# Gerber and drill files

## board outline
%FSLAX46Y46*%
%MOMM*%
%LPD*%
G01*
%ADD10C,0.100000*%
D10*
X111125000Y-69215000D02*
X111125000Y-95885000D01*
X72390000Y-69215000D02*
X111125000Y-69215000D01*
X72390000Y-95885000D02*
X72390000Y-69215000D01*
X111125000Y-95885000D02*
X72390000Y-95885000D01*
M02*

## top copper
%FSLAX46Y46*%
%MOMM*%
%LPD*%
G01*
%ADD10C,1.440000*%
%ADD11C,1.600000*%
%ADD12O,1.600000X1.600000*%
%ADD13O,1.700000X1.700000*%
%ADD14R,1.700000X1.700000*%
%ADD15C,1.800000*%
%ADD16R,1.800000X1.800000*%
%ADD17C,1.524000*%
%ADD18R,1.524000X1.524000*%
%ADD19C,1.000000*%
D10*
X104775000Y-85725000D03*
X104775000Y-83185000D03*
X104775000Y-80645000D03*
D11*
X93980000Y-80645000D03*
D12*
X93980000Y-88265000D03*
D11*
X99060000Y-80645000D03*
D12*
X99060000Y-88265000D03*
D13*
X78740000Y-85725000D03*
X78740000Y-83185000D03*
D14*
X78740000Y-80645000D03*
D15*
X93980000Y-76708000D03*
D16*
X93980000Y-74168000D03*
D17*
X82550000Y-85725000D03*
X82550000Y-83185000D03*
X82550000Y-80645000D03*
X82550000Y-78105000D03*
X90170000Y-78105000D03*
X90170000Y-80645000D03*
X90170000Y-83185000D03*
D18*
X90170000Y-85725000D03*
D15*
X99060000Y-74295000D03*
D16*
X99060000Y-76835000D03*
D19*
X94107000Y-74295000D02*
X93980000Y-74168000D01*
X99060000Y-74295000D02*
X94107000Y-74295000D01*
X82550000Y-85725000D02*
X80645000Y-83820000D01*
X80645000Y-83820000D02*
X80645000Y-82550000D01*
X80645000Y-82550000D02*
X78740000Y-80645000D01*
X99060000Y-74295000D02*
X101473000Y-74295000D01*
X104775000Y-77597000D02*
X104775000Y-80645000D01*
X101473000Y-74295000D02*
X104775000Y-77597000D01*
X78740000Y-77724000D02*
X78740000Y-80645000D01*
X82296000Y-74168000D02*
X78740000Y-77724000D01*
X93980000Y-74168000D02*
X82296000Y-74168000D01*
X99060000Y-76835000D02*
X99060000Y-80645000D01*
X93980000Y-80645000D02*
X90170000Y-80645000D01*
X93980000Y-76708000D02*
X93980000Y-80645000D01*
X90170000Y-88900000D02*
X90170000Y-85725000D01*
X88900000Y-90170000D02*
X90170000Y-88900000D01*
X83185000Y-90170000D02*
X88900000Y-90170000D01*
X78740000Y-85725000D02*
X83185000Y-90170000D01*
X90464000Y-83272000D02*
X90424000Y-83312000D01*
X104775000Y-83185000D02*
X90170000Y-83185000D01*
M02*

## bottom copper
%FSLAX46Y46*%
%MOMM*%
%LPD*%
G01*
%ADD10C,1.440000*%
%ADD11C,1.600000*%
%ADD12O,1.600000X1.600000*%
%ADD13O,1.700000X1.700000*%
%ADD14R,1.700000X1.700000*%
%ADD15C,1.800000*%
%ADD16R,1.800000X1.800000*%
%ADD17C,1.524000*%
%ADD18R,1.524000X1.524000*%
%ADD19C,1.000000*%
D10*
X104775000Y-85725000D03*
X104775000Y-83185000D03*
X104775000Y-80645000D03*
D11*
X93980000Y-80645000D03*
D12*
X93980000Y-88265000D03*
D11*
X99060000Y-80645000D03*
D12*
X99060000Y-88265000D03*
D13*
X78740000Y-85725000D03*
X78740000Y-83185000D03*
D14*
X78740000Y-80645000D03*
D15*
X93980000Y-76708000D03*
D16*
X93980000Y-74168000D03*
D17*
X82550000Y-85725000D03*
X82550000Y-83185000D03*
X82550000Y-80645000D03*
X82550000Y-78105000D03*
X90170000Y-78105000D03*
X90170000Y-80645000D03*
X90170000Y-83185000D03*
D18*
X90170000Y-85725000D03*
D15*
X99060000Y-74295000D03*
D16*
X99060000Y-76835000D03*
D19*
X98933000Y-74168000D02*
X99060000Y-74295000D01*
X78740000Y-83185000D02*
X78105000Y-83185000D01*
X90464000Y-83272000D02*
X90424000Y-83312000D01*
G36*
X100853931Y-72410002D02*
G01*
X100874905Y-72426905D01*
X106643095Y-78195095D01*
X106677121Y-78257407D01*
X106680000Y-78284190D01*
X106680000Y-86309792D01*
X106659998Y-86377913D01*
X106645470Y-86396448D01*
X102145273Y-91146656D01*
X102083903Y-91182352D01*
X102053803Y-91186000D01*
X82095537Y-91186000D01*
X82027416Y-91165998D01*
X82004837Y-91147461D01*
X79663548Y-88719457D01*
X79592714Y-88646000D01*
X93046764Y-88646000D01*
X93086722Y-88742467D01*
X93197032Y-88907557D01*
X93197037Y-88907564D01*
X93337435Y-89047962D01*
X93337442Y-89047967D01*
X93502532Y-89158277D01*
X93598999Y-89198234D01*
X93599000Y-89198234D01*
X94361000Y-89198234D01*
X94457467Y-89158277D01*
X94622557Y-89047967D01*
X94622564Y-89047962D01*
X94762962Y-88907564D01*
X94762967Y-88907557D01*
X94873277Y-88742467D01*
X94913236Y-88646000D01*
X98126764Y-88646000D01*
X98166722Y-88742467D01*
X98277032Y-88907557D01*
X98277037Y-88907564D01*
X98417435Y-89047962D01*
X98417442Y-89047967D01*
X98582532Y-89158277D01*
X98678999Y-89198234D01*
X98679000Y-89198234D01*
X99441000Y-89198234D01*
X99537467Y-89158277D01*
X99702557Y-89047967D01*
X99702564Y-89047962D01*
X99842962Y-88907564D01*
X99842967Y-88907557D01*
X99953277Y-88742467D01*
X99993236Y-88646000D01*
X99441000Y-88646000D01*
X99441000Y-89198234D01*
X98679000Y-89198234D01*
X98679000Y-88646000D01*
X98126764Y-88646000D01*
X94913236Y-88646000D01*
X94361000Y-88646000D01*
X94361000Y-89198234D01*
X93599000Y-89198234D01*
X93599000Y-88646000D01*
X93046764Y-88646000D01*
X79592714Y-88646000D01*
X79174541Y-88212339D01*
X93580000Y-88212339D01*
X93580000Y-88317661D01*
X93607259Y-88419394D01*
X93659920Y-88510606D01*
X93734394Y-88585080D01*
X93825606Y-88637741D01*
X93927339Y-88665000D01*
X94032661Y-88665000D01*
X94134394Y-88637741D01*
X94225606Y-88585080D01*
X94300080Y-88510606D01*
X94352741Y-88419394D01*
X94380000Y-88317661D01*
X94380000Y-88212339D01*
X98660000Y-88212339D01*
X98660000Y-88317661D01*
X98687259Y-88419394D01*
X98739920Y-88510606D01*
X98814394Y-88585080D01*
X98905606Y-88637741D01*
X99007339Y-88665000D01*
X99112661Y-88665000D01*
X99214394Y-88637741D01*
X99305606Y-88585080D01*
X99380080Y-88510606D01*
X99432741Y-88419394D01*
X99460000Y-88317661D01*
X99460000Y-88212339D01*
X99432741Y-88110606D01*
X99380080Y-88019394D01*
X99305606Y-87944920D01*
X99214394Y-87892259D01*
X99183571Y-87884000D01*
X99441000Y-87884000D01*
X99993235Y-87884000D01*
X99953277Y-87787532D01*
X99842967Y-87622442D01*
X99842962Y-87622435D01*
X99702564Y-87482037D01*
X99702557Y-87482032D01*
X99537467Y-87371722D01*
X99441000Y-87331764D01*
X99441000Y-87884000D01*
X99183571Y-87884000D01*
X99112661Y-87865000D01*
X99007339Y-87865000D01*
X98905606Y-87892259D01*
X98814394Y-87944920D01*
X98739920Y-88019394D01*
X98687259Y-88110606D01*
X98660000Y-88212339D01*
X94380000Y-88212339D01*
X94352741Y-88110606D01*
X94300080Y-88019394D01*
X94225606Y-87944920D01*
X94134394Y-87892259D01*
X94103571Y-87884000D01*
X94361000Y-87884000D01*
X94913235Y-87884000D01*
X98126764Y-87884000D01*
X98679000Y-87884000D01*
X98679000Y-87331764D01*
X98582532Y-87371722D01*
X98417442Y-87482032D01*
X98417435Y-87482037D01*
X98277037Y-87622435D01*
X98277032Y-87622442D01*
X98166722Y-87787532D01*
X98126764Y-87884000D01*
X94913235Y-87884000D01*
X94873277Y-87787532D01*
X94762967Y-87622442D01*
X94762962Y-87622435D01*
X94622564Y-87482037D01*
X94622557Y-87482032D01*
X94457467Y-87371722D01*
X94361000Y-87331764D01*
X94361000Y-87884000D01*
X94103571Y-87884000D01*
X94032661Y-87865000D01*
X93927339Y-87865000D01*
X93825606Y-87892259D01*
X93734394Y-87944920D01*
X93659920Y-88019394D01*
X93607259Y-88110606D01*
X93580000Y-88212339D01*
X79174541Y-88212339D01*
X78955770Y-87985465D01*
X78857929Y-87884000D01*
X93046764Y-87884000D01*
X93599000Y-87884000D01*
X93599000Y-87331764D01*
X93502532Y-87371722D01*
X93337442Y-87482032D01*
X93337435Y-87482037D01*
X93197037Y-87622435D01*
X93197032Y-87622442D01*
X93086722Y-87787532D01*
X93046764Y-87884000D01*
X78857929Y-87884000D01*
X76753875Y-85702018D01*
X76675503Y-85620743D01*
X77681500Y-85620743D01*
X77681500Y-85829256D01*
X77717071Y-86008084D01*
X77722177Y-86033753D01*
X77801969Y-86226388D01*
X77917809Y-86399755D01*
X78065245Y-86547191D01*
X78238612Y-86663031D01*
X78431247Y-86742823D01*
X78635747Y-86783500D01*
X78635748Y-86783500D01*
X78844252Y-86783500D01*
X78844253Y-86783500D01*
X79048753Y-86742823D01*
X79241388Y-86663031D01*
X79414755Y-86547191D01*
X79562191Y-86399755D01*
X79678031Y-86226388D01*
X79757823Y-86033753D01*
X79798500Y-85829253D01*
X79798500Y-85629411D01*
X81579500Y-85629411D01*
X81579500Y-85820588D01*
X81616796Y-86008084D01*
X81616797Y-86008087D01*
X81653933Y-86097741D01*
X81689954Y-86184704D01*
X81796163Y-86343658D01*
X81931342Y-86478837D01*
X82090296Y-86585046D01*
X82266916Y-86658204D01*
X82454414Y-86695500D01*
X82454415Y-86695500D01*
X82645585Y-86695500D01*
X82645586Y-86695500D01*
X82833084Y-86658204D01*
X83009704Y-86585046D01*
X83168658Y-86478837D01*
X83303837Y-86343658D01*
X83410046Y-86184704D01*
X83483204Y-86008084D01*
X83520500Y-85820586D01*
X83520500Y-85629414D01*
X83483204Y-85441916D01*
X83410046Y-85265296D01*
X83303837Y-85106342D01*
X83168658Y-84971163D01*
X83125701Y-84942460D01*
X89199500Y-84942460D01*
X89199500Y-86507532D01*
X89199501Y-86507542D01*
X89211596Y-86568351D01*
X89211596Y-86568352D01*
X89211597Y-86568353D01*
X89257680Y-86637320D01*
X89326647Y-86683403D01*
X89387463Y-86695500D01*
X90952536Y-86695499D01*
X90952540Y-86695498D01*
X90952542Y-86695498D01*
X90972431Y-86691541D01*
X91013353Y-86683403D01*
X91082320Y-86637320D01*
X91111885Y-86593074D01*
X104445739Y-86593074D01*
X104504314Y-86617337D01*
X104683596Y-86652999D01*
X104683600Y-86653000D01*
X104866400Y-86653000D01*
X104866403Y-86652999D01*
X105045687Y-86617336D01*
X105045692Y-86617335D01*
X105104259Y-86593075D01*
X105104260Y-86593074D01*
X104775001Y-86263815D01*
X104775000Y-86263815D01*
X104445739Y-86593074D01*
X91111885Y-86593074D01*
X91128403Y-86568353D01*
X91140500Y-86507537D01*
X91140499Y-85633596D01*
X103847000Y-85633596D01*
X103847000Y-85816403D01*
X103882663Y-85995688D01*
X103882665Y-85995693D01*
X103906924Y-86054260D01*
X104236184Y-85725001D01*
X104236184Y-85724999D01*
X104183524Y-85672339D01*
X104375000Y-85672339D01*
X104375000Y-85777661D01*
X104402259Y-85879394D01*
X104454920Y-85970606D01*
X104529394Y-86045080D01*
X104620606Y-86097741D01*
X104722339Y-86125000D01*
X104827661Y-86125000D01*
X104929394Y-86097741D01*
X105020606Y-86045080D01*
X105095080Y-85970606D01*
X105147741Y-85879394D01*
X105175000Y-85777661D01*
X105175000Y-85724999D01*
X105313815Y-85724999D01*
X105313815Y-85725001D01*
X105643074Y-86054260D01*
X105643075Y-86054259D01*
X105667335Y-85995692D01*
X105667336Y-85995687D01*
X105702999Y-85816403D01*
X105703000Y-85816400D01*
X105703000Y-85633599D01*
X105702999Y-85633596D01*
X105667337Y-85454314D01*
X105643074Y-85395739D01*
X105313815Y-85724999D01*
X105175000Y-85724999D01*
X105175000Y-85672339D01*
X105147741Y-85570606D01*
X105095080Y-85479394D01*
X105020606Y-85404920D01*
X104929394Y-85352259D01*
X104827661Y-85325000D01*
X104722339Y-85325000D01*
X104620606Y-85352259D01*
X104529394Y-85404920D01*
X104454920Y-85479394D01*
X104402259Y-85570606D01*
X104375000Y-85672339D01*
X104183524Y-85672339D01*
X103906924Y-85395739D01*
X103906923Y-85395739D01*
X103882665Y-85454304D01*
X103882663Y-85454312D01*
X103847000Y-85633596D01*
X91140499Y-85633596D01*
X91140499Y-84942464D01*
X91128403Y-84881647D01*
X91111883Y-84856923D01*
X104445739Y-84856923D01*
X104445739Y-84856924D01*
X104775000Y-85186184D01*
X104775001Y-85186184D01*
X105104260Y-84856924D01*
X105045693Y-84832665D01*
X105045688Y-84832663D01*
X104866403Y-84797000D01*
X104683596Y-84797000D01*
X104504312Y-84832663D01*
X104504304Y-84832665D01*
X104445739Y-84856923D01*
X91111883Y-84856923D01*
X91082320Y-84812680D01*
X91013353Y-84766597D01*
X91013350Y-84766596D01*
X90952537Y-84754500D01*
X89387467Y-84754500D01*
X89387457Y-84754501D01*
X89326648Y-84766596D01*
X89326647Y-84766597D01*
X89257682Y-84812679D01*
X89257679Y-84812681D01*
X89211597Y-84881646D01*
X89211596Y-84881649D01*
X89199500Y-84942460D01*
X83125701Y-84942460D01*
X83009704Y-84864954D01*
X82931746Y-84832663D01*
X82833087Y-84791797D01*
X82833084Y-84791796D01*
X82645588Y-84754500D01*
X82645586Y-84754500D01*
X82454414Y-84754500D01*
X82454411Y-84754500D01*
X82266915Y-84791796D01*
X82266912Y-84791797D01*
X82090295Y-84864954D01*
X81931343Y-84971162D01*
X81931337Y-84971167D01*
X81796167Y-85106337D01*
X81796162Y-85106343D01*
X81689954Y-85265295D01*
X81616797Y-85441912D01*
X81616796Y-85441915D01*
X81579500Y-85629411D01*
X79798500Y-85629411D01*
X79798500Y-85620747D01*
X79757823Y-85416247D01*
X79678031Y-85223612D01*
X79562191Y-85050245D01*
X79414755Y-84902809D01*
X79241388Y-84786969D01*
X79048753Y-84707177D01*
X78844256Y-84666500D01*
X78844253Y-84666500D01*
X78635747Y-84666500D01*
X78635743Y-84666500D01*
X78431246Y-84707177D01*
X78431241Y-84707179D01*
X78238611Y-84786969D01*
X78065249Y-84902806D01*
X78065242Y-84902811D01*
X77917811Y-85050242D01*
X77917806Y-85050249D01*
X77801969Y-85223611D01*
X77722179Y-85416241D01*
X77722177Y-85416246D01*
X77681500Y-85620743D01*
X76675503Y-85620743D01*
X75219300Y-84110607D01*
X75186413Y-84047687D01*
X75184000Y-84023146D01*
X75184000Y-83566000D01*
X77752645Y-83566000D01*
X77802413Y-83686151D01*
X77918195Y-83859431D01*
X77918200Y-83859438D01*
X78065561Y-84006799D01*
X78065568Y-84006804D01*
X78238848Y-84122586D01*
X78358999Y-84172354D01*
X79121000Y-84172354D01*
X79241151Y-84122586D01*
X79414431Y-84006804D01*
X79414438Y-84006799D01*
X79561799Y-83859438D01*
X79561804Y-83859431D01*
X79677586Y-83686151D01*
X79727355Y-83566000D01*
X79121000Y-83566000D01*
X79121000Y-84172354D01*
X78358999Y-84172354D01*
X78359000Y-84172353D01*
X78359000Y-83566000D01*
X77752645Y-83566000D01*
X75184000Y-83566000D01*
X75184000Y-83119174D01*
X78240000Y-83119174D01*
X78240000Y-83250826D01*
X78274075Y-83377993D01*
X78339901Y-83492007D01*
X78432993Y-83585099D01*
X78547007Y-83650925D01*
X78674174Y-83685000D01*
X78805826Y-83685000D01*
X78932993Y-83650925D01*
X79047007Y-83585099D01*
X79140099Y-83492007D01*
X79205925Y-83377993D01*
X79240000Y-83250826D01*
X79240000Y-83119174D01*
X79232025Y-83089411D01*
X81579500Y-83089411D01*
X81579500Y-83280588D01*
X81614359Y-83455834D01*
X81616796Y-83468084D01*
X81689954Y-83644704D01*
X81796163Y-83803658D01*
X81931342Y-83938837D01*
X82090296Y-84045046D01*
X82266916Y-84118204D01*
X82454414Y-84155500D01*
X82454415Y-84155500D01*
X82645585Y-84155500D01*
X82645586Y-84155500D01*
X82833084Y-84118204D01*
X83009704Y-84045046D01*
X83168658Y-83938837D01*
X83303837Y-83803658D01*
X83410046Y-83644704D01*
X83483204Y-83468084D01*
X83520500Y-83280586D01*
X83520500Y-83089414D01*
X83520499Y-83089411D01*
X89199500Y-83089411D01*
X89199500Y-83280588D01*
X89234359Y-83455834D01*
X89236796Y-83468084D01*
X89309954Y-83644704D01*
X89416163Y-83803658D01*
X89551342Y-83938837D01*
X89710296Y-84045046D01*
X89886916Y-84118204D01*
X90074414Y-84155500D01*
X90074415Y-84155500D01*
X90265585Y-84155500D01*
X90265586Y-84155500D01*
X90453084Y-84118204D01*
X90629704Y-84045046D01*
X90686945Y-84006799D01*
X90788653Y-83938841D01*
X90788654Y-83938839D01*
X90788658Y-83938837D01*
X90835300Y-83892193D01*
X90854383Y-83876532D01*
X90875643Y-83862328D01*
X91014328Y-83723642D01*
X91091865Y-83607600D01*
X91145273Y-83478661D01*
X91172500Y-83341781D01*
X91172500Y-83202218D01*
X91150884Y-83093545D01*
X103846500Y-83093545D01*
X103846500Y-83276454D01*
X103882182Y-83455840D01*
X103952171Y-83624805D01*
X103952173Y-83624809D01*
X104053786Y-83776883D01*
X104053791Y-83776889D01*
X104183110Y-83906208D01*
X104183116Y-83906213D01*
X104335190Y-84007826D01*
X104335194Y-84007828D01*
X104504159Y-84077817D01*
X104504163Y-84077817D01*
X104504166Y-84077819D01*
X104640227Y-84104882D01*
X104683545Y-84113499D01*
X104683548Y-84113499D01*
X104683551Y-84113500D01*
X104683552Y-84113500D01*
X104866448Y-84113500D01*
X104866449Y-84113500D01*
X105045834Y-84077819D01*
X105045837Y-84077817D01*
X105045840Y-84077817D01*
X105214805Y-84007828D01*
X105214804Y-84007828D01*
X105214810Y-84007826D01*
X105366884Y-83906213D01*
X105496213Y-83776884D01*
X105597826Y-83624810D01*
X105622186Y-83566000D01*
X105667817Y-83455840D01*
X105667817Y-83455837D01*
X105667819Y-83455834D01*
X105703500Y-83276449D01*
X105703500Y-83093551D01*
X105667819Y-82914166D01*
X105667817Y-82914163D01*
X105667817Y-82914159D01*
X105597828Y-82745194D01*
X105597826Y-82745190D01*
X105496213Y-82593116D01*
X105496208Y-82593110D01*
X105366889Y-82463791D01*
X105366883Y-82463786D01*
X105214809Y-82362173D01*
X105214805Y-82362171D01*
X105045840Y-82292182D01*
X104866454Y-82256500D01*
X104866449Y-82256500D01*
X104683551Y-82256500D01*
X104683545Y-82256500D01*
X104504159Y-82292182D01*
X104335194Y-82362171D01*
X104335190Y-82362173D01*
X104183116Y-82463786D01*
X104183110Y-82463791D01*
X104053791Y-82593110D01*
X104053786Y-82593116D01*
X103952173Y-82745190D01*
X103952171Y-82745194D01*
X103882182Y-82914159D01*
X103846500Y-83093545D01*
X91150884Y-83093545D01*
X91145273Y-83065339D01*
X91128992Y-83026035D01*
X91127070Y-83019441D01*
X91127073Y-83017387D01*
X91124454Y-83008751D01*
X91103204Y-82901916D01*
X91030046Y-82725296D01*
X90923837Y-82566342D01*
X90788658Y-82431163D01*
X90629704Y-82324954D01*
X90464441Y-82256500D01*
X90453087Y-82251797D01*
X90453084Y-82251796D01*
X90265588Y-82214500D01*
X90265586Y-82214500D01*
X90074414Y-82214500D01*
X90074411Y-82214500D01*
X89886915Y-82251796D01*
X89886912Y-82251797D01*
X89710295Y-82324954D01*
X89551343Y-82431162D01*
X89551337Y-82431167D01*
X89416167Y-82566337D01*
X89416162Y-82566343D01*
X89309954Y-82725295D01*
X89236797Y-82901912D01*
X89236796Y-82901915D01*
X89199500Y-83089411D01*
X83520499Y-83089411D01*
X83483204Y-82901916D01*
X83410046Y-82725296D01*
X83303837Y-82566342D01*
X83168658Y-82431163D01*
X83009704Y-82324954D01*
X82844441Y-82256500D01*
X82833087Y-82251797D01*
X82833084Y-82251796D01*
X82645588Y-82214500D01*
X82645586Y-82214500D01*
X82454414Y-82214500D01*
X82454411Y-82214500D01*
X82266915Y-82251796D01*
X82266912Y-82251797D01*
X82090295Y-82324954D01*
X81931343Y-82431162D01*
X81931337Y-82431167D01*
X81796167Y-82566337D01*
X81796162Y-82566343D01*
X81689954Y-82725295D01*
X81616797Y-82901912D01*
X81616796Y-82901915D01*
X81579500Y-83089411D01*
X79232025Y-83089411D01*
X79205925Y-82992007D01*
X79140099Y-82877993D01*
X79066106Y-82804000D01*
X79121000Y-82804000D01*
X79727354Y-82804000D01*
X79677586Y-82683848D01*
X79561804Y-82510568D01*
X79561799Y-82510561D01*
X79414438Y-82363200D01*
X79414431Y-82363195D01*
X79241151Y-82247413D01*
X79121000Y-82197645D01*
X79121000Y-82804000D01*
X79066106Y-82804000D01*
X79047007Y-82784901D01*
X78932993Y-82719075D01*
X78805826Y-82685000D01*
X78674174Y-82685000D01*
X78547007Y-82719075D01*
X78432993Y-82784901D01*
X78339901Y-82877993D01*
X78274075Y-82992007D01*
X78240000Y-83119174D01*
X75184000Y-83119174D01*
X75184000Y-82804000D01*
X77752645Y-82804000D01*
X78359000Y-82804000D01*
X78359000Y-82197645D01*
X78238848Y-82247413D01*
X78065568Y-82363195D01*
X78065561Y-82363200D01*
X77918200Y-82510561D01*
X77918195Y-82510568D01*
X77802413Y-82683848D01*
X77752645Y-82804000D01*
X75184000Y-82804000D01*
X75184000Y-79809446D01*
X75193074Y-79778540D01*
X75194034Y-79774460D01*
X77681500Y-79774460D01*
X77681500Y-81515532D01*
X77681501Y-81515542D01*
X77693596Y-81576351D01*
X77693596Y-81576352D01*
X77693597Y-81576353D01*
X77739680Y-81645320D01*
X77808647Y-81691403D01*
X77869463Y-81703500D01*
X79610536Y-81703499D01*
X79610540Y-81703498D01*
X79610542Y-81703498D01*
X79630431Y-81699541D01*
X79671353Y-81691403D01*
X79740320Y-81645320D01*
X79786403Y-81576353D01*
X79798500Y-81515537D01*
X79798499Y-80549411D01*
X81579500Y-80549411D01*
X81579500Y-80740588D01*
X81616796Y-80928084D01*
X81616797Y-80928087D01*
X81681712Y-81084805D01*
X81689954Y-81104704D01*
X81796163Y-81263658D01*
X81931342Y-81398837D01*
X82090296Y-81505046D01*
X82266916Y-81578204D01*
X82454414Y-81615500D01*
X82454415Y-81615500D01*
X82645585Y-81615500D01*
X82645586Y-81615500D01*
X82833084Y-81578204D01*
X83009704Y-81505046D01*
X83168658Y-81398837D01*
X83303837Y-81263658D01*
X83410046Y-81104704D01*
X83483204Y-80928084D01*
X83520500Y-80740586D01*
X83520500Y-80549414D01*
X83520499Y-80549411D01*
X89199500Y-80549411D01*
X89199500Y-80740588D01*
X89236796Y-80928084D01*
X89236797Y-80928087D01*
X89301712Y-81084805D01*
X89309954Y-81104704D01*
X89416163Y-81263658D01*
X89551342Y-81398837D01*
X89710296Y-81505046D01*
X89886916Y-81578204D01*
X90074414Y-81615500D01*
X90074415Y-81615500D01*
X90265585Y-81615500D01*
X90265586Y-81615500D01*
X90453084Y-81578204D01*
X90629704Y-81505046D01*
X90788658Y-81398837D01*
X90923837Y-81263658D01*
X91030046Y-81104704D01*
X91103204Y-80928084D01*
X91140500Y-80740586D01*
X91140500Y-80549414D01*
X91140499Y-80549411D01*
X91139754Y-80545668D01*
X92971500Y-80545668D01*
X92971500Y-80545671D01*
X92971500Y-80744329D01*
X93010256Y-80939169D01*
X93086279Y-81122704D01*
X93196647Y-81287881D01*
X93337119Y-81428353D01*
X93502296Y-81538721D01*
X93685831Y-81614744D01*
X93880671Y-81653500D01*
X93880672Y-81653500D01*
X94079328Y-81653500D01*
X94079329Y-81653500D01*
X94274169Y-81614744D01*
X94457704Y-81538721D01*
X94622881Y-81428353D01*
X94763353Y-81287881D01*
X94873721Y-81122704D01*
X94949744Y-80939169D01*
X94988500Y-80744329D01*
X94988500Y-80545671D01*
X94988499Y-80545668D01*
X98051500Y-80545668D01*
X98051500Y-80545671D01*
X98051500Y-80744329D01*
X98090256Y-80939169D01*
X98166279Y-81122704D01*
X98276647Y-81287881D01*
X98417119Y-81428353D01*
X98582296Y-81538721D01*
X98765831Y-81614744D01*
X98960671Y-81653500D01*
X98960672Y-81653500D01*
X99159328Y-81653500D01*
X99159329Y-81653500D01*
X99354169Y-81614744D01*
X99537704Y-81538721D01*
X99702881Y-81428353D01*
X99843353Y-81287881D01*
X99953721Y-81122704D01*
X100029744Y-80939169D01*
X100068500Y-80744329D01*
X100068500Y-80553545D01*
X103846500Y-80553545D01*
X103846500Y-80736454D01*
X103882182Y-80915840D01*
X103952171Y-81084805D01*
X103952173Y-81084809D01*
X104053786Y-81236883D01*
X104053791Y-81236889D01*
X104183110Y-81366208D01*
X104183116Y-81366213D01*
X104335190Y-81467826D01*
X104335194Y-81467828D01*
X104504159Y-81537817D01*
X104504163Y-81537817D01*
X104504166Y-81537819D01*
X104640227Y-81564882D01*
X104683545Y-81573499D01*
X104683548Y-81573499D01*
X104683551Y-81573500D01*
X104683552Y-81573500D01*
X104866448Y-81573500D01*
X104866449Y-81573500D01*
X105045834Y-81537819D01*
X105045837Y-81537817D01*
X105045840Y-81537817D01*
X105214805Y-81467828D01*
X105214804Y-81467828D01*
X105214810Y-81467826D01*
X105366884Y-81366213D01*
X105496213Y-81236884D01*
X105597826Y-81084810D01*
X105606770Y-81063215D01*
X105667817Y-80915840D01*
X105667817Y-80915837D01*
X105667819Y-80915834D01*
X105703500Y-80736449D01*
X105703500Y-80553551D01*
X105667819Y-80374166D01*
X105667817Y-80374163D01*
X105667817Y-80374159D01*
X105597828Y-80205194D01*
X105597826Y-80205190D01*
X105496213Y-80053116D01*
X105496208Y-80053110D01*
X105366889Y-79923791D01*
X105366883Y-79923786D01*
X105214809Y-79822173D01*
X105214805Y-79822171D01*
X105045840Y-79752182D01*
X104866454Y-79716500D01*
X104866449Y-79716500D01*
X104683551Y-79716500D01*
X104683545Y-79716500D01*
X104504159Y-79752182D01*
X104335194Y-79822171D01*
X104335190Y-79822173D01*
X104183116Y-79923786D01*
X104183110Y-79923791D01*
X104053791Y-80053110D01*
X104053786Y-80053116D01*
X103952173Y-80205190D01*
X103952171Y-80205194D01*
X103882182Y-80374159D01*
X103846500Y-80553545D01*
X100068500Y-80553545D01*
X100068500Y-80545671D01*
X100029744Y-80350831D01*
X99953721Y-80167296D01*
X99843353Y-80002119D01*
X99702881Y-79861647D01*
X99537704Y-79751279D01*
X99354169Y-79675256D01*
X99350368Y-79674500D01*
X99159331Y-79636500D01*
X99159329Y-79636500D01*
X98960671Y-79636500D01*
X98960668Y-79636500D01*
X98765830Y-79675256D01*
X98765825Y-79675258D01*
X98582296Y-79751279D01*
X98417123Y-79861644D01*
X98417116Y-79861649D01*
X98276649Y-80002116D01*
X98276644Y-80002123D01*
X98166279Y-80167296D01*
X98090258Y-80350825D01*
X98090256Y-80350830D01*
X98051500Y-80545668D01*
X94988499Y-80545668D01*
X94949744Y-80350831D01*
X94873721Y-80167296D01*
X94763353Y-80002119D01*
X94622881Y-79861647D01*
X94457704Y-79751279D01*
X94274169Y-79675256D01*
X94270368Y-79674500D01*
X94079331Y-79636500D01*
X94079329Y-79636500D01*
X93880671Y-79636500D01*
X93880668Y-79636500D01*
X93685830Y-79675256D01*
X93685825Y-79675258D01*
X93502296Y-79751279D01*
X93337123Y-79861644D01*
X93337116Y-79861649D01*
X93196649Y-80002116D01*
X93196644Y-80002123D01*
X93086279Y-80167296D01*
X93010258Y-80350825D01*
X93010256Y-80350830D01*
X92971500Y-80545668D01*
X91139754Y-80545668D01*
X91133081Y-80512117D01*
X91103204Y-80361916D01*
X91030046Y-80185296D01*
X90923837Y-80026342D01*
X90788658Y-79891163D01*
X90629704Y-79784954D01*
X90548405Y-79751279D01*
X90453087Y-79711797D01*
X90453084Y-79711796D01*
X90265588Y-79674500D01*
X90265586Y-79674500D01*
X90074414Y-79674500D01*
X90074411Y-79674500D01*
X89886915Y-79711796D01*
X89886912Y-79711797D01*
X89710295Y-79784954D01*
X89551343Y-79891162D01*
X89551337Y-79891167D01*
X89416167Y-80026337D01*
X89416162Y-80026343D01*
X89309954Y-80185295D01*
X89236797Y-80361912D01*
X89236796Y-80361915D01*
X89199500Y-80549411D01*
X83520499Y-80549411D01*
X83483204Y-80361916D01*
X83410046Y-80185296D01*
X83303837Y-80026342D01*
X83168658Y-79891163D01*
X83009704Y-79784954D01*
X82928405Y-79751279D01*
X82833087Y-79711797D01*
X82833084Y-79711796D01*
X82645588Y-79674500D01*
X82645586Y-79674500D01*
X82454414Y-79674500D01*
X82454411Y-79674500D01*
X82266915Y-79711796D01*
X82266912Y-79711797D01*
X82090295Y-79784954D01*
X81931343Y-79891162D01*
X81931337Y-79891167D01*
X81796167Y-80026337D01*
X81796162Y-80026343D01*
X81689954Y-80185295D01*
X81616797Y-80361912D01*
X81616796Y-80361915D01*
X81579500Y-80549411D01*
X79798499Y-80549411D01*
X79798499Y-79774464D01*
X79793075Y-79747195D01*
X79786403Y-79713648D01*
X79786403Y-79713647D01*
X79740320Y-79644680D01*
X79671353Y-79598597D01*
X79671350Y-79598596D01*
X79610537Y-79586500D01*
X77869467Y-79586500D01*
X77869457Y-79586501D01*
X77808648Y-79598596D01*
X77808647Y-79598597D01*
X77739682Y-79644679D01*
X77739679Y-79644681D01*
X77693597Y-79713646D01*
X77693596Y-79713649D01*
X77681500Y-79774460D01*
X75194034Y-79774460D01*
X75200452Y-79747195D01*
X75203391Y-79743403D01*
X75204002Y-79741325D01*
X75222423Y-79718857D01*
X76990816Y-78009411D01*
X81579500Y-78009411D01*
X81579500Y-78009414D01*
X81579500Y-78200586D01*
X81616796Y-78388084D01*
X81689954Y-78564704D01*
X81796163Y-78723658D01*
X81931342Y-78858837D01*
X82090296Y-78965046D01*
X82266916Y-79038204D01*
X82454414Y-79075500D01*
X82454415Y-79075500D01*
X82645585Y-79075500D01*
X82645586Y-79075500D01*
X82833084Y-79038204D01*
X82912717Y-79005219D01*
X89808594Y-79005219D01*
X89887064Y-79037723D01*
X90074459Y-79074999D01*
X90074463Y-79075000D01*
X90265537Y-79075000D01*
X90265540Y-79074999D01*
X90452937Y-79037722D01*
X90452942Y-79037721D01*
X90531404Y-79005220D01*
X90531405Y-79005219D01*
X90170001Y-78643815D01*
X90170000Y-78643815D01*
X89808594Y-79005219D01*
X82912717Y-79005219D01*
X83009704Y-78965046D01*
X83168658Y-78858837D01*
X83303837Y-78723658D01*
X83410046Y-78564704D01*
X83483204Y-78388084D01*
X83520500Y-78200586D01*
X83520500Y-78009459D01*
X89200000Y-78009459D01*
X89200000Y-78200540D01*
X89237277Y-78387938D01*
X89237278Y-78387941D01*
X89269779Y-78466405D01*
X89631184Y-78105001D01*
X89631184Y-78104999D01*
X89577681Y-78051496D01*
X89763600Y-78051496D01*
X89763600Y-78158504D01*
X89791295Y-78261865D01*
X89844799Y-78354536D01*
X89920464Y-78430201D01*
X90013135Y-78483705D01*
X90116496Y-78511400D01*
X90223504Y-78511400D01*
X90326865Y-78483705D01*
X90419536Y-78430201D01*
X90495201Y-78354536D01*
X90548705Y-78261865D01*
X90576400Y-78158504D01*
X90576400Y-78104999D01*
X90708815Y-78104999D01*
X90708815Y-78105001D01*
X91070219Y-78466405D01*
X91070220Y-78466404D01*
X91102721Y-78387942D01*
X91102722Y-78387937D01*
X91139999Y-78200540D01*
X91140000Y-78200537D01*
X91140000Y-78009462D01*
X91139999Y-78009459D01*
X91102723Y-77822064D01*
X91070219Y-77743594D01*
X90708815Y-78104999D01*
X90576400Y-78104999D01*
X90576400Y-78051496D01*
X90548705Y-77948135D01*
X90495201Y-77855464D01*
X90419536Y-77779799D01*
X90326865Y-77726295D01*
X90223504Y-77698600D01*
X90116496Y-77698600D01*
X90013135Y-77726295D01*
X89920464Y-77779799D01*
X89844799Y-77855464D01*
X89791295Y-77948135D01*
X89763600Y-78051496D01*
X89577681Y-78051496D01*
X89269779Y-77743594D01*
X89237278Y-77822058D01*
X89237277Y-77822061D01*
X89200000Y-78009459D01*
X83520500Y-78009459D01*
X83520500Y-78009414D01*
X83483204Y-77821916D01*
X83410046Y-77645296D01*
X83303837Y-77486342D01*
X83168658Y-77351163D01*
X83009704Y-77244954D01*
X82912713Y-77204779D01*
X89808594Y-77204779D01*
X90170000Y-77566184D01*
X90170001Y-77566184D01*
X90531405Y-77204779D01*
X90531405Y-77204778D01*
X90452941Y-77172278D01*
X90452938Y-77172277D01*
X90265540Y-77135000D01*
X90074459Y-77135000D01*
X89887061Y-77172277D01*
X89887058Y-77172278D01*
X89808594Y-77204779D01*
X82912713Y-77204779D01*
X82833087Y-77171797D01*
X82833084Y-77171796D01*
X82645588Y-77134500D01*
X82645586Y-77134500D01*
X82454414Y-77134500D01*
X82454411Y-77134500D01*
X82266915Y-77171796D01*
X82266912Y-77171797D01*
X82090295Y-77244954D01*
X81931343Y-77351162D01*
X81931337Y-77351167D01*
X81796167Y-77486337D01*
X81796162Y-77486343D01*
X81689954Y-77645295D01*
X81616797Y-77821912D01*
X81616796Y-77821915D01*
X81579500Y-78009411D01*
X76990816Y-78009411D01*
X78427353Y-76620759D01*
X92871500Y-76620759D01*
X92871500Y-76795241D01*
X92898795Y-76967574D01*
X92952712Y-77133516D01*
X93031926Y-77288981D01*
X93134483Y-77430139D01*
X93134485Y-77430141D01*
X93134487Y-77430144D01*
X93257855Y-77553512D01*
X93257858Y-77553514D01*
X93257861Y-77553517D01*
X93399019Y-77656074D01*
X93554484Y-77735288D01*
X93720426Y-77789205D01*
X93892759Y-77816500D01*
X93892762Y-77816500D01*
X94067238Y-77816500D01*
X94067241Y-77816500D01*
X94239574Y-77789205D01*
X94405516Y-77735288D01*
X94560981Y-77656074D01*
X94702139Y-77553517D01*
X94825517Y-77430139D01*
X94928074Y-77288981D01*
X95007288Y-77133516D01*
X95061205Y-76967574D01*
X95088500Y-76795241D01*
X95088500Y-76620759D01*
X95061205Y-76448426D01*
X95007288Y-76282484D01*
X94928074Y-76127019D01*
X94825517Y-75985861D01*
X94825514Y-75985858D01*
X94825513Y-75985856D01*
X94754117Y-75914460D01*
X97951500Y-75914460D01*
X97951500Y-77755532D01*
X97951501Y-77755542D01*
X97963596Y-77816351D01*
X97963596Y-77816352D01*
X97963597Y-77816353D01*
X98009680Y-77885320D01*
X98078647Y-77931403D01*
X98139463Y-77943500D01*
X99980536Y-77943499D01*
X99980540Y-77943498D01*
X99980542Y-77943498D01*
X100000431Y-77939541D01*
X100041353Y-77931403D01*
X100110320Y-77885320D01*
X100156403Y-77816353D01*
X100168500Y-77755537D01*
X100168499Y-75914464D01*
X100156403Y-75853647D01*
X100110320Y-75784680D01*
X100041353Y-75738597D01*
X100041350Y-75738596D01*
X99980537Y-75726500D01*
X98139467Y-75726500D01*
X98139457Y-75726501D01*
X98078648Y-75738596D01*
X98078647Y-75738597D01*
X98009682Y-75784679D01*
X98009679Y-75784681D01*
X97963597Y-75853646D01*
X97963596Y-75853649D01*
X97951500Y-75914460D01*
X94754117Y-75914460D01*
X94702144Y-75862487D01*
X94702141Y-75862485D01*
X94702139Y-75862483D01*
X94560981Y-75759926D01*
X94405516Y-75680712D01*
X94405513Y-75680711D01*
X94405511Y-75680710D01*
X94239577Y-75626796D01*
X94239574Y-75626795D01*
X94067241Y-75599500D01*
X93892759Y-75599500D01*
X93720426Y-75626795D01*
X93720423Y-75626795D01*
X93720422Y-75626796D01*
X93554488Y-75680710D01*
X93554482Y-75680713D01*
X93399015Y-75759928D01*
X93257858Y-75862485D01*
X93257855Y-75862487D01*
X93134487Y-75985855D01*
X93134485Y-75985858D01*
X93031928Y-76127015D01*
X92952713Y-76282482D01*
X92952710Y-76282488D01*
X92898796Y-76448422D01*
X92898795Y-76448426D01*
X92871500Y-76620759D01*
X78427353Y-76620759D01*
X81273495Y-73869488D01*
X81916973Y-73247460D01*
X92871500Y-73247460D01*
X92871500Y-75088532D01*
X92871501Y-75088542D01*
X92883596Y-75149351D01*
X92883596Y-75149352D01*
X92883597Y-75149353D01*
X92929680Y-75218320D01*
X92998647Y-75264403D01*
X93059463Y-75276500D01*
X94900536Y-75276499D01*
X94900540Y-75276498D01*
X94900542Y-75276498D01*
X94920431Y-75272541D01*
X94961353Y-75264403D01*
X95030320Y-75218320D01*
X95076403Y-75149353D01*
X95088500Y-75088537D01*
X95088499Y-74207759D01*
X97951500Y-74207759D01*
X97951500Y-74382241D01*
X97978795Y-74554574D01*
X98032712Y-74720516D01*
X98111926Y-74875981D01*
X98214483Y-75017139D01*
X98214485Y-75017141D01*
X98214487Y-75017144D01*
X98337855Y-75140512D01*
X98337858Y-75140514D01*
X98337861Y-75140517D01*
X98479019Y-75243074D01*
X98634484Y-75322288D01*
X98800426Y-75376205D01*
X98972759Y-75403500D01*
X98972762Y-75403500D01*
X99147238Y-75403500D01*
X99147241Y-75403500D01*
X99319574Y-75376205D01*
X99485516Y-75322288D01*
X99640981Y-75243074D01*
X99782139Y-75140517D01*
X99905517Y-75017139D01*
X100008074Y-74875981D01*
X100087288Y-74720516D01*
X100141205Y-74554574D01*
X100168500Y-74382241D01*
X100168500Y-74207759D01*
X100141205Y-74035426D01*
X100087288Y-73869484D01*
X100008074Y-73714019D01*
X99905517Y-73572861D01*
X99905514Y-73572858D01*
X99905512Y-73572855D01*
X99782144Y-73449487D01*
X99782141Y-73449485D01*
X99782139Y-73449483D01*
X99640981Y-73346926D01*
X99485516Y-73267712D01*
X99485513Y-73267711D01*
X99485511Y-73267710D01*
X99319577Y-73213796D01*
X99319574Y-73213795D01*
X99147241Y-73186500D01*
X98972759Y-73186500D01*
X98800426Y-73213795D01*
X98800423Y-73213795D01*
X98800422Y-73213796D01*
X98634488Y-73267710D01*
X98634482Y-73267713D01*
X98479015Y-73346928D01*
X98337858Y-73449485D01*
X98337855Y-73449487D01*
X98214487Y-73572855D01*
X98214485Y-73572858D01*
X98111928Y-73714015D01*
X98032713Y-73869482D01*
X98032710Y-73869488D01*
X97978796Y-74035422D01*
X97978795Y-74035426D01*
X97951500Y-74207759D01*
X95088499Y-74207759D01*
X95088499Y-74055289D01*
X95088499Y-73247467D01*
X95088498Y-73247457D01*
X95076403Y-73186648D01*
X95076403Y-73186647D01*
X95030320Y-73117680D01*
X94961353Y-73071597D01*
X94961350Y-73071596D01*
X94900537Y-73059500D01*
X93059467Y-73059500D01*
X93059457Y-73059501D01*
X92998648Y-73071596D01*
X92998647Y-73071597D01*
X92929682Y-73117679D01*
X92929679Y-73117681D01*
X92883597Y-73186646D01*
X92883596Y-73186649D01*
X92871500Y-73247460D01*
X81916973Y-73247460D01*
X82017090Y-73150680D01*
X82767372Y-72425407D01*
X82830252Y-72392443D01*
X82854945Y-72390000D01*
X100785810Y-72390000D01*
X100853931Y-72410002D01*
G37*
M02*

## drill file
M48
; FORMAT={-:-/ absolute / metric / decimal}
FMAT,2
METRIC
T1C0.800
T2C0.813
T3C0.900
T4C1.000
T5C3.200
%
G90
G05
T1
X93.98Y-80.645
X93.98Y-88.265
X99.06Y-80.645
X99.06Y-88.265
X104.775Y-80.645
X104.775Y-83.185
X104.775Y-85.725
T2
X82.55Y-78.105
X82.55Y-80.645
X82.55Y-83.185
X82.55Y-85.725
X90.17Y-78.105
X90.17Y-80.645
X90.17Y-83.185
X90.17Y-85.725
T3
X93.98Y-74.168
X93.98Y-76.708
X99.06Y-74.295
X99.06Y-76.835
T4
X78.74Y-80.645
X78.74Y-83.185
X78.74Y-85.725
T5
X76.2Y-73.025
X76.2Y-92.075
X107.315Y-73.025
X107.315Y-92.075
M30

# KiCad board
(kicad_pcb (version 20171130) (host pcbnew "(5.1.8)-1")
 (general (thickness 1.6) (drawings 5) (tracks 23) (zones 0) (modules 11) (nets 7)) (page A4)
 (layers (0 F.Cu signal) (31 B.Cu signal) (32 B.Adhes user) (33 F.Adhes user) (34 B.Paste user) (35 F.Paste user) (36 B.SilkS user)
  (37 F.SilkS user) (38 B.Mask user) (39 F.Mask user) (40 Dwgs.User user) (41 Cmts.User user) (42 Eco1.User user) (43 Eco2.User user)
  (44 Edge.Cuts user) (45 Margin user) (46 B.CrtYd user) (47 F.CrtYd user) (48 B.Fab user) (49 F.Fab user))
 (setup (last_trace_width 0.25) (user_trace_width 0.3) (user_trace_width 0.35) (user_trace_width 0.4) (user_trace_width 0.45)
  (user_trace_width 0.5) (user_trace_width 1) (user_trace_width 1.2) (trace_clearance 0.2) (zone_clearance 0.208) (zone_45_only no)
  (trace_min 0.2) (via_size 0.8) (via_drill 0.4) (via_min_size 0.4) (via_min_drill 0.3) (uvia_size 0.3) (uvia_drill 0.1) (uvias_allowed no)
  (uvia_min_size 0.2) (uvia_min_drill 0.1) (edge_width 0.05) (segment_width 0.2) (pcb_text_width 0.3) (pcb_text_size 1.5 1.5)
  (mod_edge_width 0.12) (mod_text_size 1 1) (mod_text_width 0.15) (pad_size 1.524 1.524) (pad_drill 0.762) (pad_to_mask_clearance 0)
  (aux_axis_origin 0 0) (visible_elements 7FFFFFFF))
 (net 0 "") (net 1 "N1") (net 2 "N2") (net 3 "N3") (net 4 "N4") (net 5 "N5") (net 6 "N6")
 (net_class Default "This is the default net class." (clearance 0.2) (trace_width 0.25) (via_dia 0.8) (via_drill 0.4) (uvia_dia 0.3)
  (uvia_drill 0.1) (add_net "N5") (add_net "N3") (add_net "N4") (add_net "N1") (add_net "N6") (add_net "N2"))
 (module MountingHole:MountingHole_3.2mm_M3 (layer F.Cu) (at 107.315 92.075)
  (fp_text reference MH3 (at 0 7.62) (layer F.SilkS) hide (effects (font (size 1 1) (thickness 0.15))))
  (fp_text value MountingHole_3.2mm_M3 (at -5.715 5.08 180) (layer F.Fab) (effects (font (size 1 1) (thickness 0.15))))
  (pad 1 np_thru_hole circle (at 0 0) (size 3.2 3.2) (drill 3.2) (layers *.Cu *.Mask)))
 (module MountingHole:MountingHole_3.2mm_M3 (layer F.Cu) (at 76.2 92.075)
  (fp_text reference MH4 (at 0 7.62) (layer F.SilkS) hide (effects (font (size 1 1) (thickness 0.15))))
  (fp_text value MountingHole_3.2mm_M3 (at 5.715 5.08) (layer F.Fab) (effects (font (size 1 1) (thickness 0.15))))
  (pad 1 np_thru_hole circle (at 0 0) (size 3.2 3.2) (drill 3.2) (layers *.Cu *.Mask)))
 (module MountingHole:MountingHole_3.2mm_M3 (layer F.Cu) (at 107.315 73.025)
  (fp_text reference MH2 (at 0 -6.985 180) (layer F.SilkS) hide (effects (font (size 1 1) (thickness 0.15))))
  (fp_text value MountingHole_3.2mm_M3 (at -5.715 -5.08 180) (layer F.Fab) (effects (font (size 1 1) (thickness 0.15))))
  (pad 1 np_thru_hole circle (at 0 0) (size 3.2 3.2) (drill 3.2) (layers *.Cu *.Mask)))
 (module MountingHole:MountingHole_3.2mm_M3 (layer F.Cu) (at 76.2 73.025)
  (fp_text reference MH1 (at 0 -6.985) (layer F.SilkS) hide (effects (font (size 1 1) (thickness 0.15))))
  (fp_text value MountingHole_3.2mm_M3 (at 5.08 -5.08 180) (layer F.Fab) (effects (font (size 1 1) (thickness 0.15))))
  (pad 1 np_thru_hole circle (at 0 0) (size 3.2 3.2) (drill 3.2) (layers *.Cu *.Mask)))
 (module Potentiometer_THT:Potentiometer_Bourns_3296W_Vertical (layer F.Cu) (at 104.775 80.645 90)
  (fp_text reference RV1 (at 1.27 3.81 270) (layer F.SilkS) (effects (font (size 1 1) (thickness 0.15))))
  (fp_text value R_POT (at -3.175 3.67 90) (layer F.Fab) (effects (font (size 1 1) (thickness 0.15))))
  (pad 3 thru_hole circle (at -5.08 0 90) (size 1.44 1.44) (drill 0.8) (layers *.Cu *.Mask) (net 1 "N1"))
  (pad 2 thru_hole circle (at -2.54 0 90) (size 1.44 1.44) (drill 0.8) (layers *.Cu *.Mask) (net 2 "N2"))
  (pad 1 thru_hole circle (at 0 0 90) (size 1.44 1.44) (drill 0.8) (layers *.Cu *.Mask) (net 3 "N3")))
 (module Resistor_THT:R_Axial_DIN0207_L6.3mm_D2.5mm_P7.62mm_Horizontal (layer F.Cu) (at 93.98 80.645 270)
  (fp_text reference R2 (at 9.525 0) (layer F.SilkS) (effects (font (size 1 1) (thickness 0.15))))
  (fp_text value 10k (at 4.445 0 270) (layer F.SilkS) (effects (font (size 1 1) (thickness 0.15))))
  (pad 1 thru_hole circle (at 0 0 270) (size 1.6 1.6) (drill 0.8) (layers *.Cu *.Mask) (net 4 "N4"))
  (pad 2 thru_hole oval (at 7.62 0 270) (size 1.6 1.6) (drill 0.8) (layers *.Cu *.Mask) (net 1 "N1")))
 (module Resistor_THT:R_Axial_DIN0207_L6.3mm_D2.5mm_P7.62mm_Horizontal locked (layer F.Cu) (at 99.06 80.645 270)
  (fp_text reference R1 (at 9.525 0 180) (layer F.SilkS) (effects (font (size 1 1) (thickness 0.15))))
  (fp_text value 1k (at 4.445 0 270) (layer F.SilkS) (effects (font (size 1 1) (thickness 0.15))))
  (pad 1 thru_hole circle (at 0 0 270) (size 1.6 1.6) (drill 0.8) (layers *.Cu *.Mask) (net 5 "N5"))
  (pad 2 thru_hole oval (at 7.62 0 270) (size 1.6 1.6) (drill 0.8) (layers *.Cu *.Mask) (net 1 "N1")))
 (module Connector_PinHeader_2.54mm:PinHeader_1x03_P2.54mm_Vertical (layer F.Cu) (at 78.74 80.645)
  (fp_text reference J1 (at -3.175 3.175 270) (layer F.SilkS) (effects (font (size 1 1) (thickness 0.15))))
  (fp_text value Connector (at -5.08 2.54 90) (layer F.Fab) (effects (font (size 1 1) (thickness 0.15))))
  (pad 3 thru_hole oval (at 0 5.08) (size 1.7 1.7) (drill 1) (layers *.Cu *.Mask) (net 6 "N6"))
  (pad 2 thru_hole oval (at 0 2.54) (size 1.7 1.7) (drill 1) (layers *.Cu *.Mask) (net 1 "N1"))
  (pad 1 thru_hole rect (at 0 0) (size 1.7 1.7) (drill 1) (layers *.Cu *.Mask) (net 3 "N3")))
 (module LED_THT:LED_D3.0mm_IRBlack (layer F.Cu) (at 93.98 74.168 270)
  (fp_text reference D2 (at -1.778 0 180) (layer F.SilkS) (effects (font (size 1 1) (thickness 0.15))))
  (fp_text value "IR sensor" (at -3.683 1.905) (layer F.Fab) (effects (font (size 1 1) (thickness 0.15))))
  (pad 2 thru_hole circle (at 2.54 0 270) (size 1.8 1.8) (drill 0.9) (layers *.Cu *.Mask) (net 4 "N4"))
  (pad 1 thru_hole rect (at 0 0 270) (size 1.8 1.8) (drill 0.9) (layers *.Cu *.Mask) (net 3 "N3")))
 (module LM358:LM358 (layer F.Cu) (at 82.55 78.105 180)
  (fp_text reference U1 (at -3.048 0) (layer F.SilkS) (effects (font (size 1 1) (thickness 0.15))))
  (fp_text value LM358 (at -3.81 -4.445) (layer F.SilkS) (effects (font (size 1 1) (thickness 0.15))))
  (pad 8 thru_hole circle (at 0 -7.62 180) (size 1.524 1.524) (drill 0.8128) (layers *.Cu *.Mask) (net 3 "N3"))
  (pad 7 thru_hole circle (at 0 -5.08 180) (size 1.524 1.524) (drill 0.8128) (layers *.Cu *.Mask))
  (pad 6 thru_hole circle (at 0 -2.54 180) (size 1.524 1.524) (drill 0.8128) (layers *.Cu *.Mask))
  (pad 5 thru_hole circle (at 0 0 180) (size 1.524 1.524) (drill 0.8128) (layers *.Cu *.Mask))
  (pad 4 thru_hole circle (at -7.62 0 180) (size 1.524 1.524) (drill 0.8128) (layers *.Cu *.Mask) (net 1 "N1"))
  (pad 3 thru_hole circle (at -7.62 -2.54 180) (size 1.524 1.524) (drill 0.8128) (layers *.Cu *.Mask) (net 4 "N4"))
  (pad 2 thru_hole circle (at -7.62 -5.08 180) (size 1.524 1.524) (drill 0.8128) (layers *.Cu *.Mask) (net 2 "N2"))
  (pad 1 thru_hole rect (at -7.62 -7.62 180) (size 1.524 1.524) (drill 0.8128) (layers *.Cu *.Mask) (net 6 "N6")))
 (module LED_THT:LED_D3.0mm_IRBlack (layer F.Cu) (at 99.06 76.835 90)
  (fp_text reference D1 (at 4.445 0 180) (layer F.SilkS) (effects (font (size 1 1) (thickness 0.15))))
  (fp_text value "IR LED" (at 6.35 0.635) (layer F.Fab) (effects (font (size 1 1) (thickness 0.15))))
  (pad 2 thru_hole circle (at 2.54 0 90) (size 1.8 1.8) (drill 0.9) (layers *.Cu *.Mask) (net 3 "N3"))
  (pad 1 thru_hole rect (at 0 0 90) (size 1.8 1.8) (drill 0.9) (layers *.Cu *.Mask) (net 5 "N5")))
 (gr_line (start 111.125 69.215) (end 111.125 95.885) (layer Edge.Cuts) (width 0.1))
 (gr_line (start 72.39 69.215) (end 111.125 69.215) (layer Edge.Cuts) (width 0.1))
 (gr_line (start 72.39 95.885) (end 72.39 69.215) (layer Edge.Cuts) (width 0.1))
 (gr_line (start 111.125 95.885) (end 72.39 95.885) (layer Edge.Cuts) (width 0.1))
 (segment (start 98.933 74.168) (end 99.06 74.295) (width 1) (layer B.Cu) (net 3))
 (segment (start 94.107 74.295) (end 93.98 74.168) (width 1) (layer F.Cu) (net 3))
 (segment (start 99.06 74.295) (end 94.107 74.295) (width 1) (layer F.Cu) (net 3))
 (segment (start 82.55 85.725) (end 80.645 83.82) (width 1) (layer F.Cu) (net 3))
 (segment (start 80.645 83.82) (end 80.645 82.55) (width 1) (layer F.Cu) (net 3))
 (segment (start 80.645 82.55) (end 78.74 80.645) (width 1) (layer F.Cu) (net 3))
 (segment (start 99.06 74.295) (end 101.473 74.295) (width 1) (layer F.Cu) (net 3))
 (segment (start 104.775 77.597) (end 104.775 80.645) (width 1) (layer F.Cu) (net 3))
 (segment (start 101.473 74.295) (end 104.775 77.597) (width 1) (layer F.Cu) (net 3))
 (segment (start 78.74 77.724) (end 78.74 80.645) (width 1) (layer F.Cu) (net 3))
 (segment (start 82.296 74.168) (end 78.74 77.724) (width 1) (layer F.Cu) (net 3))
 (segment (start 93.98 74.168) (end 82.296 74.168) (width 1) (layer F.Cu) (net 3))
 (segment (start 99.06 76.835) (end 99.06 80.645) (width 1) (layer F.Cu) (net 5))
 (segment (start 93.98 80.645) (end 90.17 80.645) (width 1) (layer F.Cu) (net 4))
 (segment (start 93.98 76.708) (end 93.98 80.645) (width 1) (layer F.Cu) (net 4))
 (segment (start 90.17 88.9) (end 90.17 85.725) (width 1) (layer F.Cu) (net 6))
 (segment (start 88.9 90.17) (end 90.17 88.9) (width 1) (layer F.Cu) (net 6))
 (segment (start 83.185 90.17) (end 88.9 90.17) (width 1) (layer F.Cu) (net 6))
 (segment (start 78.74 85.725) (end 83.185 90.17) (width 1) (layer F.Cu) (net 6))
 (segment (start 78.74 83.185) (end 78.105 83.185) (width 1) (layer B.Cu) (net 1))
 (segment (start 90.464 83.272) (end 90.424 83.312) (width 1) (layer F.Cu) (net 2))
 (segment (start 90.464 83.272) (end 90.424 83.312) (width 1) (layer B.Cu) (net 2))
 (segment (start 104.775 83.185) (end 90.17 83.185) (width 1) (layer F.Cu) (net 2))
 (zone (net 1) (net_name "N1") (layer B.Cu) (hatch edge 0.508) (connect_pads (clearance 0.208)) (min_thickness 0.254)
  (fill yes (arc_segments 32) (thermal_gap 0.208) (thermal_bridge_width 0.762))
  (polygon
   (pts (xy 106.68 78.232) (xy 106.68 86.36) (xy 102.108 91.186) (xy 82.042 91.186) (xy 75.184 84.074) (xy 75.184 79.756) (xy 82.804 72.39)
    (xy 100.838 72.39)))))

